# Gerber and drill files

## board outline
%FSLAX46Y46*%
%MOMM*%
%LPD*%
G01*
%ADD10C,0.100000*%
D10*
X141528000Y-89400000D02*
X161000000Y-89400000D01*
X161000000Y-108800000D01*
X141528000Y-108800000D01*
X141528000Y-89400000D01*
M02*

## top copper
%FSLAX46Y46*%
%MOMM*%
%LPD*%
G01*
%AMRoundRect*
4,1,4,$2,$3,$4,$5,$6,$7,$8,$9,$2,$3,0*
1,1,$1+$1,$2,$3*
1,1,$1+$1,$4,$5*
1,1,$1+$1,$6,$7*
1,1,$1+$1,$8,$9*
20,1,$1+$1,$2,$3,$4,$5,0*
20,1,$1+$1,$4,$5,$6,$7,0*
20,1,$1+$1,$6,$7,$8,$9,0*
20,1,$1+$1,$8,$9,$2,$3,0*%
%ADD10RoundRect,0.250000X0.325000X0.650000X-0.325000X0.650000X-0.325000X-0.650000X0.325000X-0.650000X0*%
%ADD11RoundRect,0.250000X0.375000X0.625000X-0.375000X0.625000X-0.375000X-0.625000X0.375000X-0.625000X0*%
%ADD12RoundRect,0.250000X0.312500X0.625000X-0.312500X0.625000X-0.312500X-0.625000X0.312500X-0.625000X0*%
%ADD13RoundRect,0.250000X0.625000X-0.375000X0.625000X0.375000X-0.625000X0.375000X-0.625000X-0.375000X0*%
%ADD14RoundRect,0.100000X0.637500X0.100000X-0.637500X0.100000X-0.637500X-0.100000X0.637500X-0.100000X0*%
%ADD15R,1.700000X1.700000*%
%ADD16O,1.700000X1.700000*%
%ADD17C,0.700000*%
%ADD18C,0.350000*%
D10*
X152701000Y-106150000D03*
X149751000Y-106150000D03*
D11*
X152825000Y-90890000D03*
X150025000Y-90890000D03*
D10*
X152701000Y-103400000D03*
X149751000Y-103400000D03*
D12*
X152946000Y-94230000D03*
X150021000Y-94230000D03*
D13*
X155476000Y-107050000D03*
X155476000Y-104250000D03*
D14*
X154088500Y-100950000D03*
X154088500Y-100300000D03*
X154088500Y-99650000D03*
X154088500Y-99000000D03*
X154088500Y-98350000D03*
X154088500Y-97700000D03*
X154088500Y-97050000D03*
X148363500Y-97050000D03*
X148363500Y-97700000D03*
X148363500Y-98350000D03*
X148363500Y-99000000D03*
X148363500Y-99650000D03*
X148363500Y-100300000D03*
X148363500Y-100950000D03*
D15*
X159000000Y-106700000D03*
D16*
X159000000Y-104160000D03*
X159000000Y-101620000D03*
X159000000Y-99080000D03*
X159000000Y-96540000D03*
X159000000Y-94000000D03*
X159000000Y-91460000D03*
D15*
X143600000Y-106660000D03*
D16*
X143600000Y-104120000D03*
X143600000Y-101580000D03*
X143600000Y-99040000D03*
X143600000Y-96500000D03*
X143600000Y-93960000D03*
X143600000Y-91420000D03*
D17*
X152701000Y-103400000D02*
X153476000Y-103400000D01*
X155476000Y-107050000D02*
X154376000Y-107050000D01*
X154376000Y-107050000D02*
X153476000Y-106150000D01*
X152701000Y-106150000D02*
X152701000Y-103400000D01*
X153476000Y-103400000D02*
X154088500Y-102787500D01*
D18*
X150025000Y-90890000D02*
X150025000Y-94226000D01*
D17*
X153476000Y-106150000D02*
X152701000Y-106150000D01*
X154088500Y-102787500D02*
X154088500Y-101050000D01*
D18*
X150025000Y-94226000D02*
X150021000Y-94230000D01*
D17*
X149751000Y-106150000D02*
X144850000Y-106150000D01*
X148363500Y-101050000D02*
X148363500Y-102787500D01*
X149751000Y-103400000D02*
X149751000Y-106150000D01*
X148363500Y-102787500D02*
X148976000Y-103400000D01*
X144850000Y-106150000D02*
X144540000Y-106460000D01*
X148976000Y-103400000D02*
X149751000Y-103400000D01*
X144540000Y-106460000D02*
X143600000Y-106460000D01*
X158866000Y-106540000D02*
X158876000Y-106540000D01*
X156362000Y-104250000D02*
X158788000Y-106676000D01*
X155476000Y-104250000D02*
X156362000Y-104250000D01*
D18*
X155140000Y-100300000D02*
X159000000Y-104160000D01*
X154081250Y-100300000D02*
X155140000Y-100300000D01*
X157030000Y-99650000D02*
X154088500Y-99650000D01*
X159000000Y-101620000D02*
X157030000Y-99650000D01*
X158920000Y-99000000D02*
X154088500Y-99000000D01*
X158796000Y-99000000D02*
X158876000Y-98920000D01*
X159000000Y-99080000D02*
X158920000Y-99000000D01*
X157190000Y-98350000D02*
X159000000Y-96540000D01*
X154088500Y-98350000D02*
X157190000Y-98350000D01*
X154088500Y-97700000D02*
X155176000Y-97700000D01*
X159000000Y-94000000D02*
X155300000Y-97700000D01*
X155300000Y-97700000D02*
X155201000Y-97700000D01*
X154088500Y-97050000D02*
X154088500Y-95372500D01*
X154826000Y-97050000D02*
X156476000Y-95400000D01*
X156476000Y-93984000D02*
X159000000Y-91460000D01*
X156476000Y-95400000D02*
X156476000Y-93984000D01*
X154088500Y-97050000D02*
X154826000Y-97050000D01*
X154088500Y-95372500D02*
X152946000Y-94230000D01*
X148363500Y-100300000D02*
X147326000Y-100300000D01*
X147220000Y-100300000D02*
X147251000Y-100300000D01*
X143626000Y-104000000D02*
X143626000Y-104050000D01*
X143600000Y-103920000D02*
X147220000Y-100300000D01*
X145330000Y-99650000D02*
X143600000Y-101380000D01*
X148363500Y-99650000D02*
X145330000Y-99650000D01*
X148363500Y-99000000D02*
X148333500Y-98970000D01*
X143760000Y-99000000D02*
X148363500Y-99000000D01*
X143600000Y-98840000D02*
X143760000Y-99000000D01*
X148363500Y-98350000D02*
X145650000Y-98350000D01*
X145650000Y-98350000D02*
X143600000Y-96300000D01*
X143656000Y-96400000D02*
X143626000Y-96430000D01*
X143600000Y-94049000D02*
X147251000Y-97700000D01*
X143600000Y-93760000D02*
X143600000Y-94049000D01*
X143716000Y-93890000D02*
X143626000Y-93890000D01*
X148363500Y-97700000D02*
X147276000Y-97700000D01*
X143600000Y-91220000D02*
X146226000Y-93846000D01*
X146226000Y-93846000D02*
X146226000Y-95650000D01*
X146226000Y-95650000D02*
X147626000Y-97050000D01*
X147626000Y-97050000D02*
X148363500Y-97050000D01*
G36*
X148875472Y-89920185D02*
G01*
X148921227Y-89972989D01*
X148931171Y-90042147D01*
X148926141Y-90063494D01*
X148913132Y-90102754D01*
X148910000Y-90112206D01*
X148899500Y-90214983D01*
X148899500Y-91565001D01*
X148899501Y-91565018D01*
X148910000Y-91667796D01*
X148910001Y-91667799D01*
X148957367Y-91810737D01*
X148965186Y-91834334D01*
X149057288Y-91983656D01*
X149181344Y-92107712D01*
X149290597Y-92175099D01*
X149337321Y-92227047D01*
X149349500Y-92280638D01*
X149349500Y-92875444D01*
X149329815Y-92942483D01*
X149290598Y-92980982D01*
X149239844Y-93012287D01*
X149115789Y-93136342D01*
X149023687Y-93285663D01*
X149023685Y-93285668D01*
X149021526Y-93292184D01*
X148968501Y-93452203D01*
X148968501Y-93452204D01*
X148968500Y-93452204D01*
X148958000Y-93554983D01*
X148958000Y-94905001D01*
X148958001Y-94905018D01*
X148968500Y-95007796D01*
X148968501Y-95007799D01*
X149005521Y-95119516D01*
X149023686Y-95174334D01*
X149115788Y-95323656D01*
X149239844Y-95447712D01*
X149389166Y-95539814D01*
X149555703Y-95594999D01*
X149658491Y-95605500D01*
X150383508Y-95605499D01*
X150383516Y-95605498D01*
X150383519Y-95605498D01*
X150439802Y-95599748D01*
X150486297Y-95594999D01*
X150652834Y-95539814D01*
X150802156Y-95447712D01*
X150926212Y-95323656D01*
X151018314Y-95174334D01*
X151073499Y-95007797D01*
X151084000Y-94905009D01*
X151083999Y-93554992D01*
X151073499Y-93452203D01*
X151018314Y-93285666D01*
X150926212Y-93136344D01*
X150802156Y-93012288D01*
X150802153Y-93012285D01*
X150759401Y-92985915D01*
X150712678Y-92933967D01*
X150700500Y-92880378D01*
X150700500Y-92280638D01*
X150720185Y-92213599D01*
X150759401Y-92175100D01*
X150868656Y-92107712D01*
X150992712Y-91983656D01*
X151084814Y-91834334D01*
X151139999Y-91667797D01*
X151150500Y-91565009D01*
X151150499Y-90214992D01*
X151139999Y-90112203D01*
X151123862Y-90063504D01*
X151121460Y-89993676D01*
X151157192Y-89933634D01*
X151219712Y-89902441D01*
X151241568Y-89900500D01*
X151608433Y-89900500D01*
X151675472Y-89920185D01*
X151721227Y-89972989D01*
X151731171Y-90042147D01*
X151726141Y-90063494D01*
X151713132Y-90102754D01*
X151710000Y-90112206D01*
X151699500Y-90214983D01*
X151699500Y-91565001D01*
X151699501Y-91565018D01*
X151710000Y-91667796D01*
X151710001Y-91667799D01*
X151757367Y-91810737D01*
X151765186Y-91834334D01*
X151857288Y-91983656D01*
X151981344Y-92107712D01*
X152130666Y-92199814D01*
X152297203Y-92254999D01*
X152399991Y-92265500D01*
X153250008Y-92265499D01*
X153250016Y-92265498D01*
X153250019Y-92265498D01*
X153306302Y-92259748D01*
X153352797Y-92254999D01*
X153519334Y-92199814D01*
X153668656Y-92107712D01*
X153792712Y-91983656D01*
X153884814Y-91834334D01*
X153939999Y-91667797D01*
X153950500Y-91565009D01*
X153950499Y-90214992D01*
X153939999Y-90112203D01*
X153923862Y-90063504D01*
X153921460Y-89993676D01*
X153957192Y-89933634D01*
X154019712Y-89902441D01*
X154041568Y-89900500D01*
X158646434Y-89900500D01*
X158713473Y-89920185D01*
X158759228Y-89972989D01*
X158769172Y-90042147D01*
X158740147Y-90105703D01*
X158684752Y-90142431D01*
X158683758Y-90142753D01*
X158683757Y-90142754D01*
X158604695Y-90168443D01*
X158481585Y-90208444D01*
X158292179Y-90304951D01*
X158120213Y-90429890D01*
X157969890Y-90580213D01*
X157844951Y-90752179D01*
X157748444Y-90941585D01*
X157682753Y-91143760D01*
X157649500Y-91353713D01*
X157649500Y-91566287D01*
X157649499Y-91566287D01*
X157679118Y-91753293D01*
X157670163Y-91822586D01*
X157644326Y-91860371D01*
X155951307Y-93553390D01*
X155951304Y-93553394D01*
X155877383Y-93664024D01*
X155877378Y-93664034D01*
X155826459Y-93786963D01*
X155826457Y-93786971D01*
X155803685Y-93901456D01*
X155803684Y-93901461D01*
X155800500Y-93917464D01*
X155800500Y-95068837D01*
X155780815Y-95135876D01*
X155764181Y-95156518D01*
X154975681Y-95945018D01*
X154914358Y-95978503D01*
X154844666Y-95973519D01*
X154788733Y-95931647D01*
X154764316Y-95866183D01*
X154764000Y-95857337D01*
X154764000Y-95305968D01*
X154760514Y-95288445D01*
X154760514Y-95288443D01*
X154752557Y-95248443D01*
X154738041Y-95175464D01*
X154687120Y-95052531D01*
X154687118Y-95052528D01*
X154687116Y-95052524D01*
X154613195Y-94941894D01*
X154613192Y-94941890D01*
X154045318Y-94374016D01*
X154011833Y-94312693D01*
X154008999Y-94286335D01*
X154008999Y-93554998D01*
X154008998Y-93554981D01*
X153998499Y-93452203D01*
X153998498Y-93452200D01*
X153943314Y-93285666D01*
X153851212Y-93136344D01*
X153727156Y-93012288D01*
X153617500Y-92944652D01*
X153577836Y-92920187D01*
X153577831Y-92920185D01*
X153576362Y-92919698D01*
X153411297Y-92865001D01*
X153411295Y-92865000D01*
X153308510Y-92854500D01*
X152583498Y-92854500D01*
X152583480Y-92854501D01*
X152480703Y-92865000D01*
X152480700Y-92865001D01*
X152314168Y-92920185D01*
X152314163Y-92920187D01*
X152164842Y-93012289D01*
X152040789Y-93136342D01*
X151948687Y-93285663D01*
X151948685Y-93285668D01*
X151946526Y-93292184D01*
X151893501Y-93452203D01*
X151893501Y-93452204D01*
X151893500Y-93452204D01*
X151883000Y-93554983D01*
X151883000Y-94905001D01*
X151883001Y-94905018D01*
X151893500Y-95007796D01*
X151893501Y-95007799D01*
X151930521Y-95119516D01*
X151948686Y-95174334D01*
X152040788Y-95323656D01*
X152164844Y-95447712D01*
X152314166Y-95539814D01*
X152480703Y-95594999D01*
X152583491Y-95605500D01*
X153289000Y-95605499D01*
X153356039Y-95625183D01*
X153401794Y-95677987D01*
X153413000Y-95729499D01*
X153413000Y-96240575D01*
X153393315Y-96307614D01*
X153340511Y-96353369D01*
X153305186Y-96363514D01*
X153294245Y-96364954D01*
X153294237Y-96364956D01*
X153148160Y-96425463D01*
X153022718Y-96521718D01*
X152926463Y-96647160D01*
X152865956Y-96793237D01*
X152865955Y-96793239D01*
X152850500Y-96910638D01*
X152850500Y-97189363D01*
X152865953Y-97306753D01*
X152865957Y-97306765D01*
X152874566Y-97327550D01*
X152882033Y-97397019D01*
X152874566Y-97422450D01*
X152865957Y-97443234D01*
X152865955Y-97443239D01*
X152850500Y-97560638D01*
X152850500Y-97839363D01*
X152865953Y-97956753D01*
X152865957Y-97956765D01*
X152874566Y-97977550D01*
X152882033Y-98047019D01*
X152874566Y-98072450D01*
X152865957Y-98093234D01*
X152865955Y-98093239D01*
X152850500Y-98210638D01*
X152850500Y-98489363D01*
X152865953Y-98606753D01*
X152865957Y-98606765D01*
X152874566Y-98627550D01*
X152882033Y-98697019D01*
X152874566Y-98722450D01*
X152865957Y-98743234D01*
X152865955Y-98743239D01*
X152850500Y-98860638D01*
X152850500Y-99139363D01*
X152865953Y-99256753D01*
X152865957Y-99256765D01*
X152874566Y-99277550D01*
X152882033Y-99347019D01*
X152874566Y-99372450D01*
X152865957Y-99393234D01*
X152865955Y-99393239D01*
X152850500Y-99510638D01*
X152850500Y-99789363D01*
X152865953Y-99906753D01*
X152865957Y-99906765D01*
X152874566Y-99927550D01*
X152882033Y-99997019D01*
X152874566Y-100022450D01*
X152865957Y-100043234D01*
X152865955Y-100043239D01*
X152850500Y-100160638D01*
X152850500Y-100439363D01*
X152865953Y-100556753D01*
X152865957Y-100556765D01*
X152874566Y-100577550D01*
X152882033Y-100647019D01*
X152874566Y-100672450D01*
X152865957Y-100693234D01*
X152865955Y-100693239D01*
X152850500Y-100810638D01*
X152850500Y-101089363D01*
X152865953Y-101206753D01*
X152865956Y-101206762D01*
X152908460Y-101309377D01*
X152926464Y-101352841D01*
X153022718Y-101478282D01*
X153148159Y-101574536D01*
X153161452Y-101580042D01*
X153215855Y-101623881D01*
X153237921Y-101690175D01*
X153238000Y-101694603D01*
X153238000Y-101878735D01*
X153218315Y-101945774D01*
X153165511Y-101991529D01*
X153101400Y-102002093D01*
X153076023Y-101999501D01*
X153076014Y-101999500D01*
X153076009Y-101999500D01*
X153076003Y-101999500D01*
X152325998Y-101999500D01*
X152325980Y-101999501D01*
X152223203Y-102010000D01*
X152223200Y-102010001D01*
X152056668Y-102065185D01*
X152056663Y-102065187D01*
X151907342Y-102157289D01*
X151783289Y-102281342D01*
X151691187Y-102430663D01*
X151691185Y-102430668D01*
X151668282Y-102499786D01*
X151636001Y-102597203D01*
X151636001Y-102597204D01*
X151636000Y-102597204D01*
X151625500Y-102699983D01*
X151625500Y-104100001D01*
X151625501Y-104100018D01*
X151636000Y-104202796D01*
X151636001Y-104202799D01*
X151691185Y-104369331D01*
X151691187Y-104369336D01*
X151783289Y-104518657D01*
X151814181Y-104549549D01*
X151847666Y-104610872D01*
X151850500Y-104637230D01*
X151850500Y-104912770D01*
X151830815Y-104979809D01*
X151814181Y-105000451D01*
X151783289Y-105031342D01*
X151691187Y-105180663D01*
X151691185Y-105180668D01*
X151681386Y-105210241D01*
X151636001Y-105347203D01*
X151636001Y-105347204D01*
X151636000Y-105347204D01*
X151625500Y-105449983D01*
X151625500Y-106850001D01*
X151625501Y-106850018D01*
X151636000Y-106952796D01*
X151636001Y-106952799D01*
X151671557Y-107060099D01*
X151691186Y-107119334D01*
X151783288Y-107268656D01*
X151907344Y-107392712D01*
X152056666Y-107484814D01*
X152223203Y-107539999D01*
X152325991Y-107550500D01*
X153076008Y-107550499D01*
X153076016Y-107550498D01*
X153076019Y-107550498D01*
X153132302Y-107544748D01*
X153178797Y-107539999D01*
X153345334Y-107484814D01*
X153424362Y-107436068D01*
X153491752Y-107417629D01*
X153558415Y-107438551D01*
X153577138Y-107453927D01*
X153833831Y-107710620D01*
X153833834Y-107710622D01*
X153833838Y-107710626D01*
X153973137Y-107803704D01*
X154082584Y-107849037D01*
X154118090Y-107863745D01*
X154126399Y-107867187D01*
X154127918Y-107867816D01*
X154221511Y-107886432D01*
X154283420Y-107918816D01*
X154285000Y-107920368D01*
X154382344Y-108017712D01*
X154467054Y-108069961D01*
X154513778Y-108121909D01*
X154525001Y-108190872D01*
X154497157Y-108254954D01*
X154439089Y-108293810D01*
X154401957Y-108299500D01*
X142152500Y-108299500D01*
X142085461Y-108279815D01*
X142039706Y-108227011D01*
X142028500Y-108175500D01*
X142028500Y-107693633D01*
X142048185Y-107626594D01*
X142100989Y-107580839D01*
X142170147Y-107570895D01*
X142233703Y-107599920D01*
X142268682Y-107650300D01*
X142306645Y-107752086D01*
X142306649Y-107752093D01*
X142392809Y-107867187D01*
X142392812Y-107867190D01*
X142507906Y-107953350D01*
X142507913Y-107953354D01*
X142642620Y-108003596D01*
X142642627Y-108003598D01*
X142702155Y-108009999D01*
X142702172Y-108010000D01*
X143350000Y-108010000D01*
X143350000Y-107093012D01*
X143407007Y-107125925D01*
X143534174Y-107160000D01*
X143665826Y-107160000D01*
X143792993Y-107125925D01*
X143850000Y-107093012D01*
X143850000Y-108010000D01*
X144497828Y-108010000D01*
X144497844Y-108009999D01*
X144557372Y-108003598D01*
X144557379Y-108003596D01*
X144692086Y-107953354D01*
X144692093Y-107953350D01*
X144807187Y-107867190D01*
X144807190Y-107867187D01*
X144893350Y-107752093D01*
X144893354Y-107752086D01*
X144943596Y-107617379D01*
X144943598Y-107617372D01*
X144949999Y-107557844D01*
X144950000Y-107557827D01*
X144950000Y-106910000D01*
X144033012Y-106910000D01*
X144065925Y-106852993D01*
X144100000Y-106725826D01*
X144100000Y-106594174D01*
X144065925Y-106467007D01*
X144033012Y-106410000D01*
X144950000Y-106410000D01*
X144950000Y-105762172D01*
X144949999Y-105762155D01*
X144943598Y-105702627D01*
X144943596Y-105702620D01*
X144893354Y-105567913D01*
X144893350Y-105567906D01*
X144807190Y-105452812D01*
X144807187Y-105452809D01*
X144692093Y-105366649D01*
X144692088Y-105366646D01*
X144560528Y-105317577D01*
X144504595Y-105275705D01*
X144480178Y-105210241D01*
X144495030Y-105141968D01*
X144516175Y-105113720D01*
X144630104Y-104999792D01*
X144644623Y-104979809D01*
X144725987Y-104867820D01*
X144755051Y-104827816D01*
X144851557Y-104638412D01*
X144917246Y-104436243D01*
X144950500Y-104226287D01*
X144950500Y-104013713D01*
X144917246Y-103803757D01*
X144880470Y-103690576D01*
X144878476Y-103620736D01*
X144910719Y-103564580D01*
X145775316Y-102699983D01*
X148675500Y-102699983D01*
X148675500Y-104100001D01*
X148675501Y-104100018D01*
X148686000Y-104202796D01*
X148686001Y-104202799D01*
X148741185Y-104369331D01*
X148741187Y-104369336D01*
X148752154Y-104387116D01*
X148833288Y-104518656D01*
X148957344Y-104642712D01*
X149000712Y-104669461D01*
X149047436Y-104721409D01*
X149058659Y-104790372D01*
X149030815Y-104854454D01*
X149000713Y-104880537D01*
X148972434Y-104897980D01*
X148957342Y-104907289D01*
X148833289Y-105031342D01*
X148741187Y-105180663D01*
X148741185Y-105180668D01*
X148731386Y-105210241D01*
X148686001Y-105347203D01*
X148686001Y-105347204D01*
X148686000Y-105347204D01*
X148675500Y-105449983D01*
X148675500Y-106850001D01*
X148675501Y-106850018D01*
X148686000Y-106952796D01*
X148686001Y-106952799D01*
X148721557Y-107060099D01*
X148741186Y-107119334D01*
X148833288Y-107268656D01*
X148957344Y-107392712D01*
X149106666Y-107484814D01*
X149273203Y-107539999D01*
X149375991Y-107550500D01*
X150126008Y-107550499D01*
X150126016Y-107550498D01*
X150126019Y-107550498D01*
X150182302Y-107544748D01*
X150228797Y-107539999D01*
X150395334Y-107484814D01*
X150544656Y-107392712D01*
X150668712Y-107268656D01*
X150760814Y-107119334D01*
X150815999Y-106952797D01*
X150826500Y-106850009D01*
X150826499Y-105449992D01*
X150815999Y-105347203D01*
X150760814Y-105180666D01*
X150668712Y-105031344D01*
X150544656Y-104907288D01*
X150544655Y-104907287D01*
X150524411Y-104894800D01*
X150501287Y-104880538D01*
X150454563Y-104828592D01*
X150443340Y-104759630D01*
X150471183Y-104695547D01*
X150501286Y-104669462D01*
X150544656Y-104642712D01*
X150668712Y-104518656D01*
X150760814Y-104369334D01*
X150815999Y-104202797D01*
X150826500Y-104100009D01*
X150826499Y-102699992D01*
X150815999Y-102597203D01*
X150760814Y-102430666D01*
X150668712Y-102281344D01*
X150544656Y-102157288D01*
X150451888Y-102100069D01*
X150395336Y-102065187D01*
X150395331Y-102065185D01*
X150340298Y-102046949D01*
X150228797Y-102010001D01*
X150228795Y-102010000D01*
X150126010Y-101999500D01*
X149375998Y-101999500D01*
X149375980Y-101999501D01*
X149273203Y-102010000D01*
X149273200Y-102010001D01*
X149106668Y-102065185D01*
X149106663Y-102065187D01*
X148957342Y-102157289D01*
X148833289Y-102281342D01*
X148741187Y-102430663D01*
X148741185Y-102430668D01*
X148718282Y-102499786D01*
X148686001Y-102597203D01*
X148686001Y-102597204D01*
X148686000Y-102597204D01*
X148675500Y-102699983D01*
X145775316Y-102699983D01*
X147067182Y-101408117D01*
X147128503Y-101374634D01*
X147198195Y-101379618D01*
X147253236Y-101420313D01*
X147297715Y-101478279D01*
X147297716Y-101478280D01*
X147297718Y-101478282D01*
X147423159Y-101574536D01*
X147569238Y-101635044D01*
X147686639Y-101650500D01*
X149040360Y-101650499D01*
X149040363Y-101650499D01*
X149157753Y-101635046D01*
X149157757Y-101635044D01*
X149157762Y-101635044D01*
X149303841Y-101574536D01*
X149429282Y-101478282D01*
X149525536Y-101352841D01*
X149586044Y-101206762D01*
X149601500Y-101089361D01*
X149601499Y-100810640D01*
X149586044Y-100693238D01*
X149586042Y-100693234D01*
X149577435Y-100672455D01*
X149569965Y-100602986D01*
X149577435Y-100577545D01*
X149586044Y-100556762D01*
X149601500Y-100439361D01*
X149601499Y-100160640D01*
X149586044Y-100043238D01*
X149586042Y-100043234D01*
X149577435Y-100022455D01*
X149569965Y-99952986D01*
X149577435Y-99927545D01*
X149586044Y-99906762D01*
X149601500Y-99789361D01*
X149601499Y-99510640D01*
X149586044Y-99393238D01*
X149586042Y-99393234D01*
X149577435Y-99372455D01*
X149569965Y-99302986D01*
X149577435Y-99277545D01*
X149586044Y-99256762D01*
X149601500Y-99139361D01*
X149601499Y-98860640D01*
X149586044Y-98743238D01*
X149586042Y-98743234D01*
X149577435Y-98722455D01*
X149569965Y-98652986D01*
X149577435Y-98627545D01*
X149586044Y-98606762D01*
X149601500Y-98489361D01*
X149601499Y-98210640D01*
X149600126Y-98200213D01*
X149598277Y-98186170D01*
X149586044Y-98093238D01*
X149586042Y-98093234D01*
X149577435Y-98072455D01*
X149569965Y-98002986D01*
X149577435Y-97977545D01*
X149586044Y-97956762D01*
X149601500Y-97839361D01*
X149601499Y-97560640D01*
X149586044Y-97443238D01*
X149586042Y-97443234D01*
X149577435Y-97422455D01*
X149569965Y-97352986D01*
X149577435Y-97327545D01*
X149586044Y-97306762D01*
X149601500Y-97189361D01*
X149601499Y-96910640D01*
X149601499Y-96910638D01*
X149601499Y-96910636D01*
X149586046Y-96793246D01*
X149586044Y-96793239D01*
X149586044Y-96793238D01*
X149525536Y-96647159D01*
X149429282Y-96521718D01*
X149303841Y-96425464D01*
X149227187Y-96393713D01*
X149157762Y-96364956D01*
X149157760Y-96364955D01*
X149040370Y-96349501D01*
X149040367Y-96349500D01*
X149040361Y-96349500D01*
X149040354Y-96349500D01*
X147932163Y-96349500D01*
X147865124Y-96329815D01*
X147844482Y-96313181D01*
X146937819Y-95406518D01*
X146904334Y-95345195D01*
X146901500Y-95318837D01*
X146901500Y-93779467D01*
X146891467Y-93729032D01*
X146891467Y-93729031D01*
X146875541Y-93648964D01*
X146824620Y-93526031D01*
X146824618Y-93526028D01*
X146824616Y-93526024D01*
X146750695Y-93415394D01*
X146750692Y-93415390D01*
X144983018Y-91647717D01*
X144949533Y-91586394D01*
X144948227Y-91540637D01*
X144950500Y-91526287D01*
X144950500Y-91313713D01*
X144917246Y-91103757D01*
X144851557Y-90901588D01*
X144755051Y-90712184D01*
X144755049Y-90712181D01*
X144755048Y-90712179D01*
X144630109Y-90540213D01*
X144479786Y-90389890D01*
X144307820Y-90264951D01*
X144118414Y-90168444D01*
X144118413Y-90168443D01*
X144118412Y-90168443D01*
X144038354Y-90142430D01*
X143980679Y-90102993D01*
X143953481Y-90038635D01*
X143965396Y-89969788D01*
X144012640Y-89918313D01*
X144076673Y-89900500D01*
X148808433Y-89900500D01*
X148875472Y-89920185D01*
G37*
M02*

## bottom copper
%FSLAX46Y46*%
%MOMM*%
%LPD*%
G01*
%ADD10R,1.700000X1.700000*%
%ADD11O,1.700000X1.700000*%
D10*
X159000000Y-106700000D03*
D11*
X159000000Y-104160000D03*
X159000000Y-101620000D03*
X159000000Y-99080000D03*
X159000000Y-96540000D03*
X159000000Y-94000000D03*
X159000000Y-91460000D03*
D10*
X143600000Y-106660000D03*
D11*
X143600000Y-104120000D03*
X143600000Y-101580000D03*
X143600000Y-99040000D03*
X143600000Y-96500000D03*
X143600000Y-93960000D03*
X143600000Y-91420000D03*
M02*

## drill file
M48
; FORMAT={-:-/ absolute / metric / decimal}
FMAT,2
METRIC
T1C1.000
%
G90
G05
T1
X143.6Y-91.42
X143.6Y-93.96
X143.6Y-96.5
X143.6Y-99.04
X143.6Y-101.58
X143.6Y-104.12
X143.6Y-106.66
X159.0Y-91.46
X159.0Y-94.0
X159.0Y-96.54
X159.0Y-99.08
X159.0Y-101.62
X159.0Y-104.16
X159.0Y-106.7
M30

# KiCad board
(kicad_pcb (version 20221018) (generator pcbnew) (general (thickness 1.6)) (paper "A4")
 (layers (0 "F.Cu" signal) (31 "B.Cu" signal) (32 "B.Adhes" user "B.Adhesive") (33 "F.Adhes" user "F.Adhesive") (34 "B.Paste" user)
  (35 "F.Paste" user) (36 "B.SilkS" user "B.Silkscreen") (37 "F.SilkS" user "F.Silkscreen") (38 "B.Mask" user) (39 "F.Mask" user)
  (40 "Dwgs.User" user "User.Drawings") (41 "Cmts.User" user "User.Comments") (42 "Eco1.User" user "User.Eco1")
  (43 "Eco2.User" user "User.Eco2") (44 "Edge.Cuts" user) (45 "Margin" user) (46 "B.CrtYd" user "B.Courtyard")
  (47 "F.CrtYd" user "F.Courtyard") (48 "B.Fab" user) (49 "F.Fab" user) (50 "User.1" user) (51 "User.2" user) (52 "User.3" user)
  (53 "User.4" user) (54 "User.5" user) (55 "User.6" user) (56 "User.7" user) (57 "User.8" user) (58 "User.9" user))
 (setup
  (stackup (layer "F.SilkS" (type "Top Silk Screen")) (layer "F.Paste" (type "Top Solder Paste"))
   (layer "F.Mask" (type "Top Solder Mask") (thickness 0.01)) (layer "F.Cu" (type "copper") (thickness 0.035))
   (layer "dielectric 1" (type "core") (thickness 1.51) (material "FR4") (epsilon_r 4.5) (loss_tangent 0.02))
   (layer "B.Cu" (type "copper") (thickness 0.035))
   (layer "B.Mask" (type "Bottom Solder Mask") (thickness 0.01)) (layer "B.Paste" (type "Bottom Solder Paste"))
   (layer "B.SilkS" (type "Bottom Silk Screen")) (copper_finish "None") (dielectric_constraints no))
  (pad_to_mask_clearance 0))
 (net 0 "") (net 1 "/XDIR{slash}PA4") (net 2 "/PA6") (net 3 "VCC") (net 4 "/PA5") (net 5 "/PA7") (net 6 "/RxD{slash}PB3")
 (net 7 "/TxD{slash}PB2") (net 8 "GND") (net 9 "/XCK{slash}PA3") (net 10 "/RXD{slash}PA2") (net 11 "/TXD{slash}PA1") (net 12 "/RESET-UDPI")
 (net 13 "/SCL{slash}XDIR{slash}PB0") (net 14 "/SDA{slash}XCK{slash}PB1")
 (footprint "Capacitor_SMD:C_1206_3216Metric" (layer "F.Cu") (at 151.226 106.15 180)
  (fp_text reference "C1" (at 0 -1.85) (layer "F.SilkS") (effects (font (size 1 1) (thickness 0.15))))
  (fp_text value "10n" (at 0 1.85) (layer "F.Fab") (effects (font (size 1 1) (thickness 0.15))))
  (pad "1" smd roundrect (at -1.475 0 180) (size 1.15 1.8) (layers "F.Cu" "F.Paste" "F.Mask") (roundrect_rratio 0.2173913043))
  (pad "2" smd roundrect (at 1.475 0 180) (size 1.15 1.8) (layers "F.Cu" "F.Paste" "F.Mask") (roundrect_rratio 0.2173913043)))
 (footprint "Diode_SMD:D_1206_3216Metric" (layer "F.Cu") (at 151.425 90.89 180)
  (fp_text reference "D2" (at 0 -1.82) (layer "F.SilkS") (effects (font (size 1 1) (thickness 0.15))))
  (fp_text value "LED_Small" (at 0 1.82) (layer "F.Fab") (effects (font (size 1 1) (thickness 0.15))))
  (pad "1" smd roundrect (at -1.4 0 180) (size 1.25 1.75) (layers "F.Cu" "F.Paste" "F.Mask") (roundrect_rratio 0.2))
  (pad "2" smd roundrect (at 1.4 0 180) (size 1.25 1.75) (layers "F.Cu" "F.Paste" "F.Mask") (roundrect_rratio 0.2)))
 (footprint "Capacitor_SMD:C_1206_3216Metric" (layer "F.Cu") (at 151.226 103.4 180)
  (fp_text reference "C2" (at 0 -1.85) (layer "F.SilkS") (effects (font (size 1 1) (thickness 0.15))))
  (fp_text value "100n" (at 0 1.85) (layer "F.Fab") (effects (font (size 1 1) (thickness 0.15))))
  (pad "1" smd roundrect (at -1.475 0 180) (size 1.15 1.8) (layers "F.Cu" "F.Paste" "F.Mask") (roundrect_rratio 0.2173913043))
  (pad "2" smd roundrect (at 1.475 0 180) (size 1.15 1.8) (layers "F.Cu" "F.Paste" "F.Mask") (roundrect_rratio 0.2173913043)))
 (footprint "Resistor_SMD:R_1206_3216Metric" (layer "F.Cu") (at 151.4835 94.23 180)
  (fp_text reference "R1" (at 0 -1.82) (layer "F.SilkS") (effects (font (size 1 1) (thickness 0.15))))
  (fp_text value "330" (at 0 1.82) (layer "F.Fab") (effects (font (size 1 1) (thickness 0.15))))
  (pad "1" smd roundrect (at -1.4625 0 180) (size 1.125 1.75) (layers "F.Cu" "F.Paste" "F.Mask") (roundrect_rratio 0.2222222222))
  (pad "2" smd roundrect (at 1.4625 0 180) (size 1.125 1.75) (layers "F.Cu" "F.Paste" "F.Mask") (roundrect_rratio 0.2222222222)))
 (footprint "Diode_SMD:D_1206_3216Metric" (layer "F.Cu") (at 155.476 105.65 90)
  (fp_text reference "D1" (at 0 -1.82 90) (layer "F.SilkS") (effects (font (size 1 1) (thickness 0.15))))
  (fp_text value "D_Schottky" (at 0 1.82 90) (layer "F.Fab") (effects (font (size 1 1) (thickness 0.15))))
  (pad "1" smd roundrect (at -1.4 0 90) (size 1.25 1.75) (layers "F.Cu" "F.Paste" "F.Mask") (roundrect_rratio 0.2))
  (pad "2" smd roundrect (at 1.4 0 90) (size 1.25 1.75) (layers "F.Cu" "F.Paste" "F.Mask") (roundrect_rratio 0.2)))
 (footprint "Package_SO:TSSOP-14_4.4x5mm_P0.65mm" (layer "F.Cu") (at 151.226 99 180)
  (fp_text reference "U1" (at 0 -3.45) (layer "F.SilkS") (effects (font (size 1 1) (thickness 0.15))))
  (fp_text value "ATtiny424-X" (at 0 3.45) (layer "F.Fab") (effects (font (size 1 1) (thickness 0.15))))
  (pad "1" smd roundrect (at -2.8625 -1.95 180) (size 1.475 0.4) (layers "F.Cu" "F.Paste" "F.Mask") (roundrect_rratio 0.25))
  (pad "2" smd roundrect (at -2.8625 -1.3 180) (size 1.475 0.4) (layers "F.Cu" "F.Paste" "F.Mask") (roundrect_rratio 0.25)
   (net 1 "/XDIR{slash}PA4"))
  (pad "3" smd roundrect (at -2.8625 -0.65 180) (size 1.475 0.4) (layers "F.Cu" "F.Paste" "F.Mask") (roundrect_rratio 0.25))
  (pad "4" smd roundrect (at -2.8625 0 180) (size 1.475 0.4) (layers "F.Cu" "F.Paste" "F.Mask") (roundrect_rratio 0.25) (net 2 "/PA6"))
  (pad "5" smd roundrect (at -2.8625 0.65 180) (size 1.475 0.4) (layers "F.Cu" "F.Paste" "F.Mask") (roundrect_rratio 0.25))
  (pad "6" smd roundrect (at -2.8625 1.3 180) (size 1.475 0.4) (layers "F.Cu" "F.Paste" "F.Mask") (roundrect_rratio 0.25))
  (pad "7" smd roundrect (at -2.8625 1.95 180) (size 1.475 0.4) (layers "F.Cu" "F.Paste" "F.Mask") (roundrect_rratio 0.25))
  (pad "8" smd roundrect (at 2.8625 1.95 180) (size 1.475 0.4) (layers "F.Cu" "F.Paste" "F.Mask") (roundrect_rratio 0.25))
  (pad "9" smd roundrect (at 2.8625 1.3 180) (size 1.475 0.4) (layers "F.Cu" "F.Paste" "F.Mask") (roundrect_rratio 0.25))
  (pad "10" smd roundrect (at 2.8625 0.65 180) (size 1.475 0.4) (layers "F.Cu" "F.Paste" "F.Mask") (roundrect_rratio 0.25))
  (pad "11" smd roundrect (at 2.8625 0 180) (size 1.475 0.4) (layers "F.Cu" "F.Paste" "F.Mask") (roundrect_rratio 0.25))
  (pad "12" smd roundrect (at 2.8625 -0.65 180) (size 1.475 0.4) (layers "F.Cu" "F.Paste" "F.Mask") (roundrect_rratio 0.25))
  (pad "13" smd roundrect (at 2.8625 -1.3 180) (size 1.475 0.4) (layers "F.Cu" "F.Paste" "F.Mask") (roundrect_rratio 0.25))
  (pad "14" smd roundrect (at 2.8625 -1.95 180) (size 1.475 0.4) (layers "F.Cu" "F.Paste" "F.Mask") (roundrect_rratio 0.25)))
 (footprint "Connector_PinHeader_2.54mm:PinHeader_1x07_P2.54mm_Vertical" (layer "B.Cu") (at 159 106.7)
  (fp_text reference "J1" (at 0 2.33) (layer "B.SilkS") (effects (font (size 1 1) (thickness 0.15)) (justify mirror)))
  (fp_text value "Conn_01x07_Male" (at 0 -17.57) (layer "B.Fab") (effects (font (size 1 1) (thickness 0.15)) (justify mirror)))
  (pad "1" thru_hole rect (at 0 0) (size 1.7 1.7) (drill 1) (layers "*.Cu" "*.Mask") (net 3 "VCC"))
  (pad "2" thru_hole oval (at 0 -2.54) (size 1.7 1.7) (drill 1) (layers "*.Cu" "*.Mask") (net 1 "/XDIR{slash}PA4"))
  (pad "3" thru_hole oval (at 0 -5.08) (size 1.7 1.7) (drill 1) (layers "*.Cu" "*.Mask") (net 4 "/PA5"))
  (pad "4" thru_hole oval (at 0 -7.62) (size 1.7 1.7) (drill 1) (layers "*.Cu" "*.Mask") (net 2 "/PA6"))
  (pad "5" thru_hole oval (at 0 -10.16) (size 1.7 1.7) (drill 1) (layers "*.Cu" "*.Mask") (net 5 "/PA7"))
  (pad "6" thru_hole oval (at 0 -12.7) (size 1.7 1.7) (drill 1) (layers "*.Cu" "*.Mask") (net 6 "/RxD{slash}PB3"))
  (pad "7" thru_hole oval (at 0 -15.24) (size 1.7 1.7) (drill 1) (layers "*.Cu" "*.Mask") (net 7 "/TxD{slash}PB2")))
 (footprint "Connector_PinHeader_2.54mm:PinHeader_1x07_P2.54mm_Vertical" (layer "B.Cu") (at 143.6 106.66)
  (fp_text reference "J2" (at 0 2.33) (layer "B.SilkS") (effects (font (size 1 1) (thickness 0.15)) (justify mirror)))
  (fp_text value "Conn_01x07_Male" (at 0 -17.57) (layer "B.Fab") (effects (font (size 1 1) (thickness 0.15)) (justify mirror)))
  (pad "1" thru_hole rect (at 0 0) (size 1.7 1.7) (drill 1) (layers "*.Cu" "*.Mask") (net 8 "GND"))
  (pad "2" thru_hole oval (at 0 -2.54) (size 1.7 1.7) (drill 1) (layers "*.Cu" "*.Mask") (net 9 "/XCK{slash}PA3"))
  (pad "3" thru_hole oval (at 0 -5.08) (size 1.7 1.7) (drill 1) (layers "*.Cu" "*.Mask") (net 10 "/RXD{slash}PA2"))
  (pad "4" thru_hole oval (at 0 -7.62) (size 1.7 1.7) (drill 1) (layers "*.Cu" "*.Mask") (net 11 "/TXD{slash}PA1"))
  (pad "5" thru_hole oval (at 0 -10.16) (size 1.7 1.7) (drill 1) (layers "*.Cu" "*.Mask") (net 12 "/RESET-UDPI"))
  (pad "6" thru_hole oval (at 0 -12.7) (size 1.7 1.7) (drill 1) (layers "*.Cu" "*.Mask") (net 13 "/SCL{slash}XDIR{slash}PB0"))
  (pad "7" thru_hole oval (at 0 -15.24) (size 1.7 1.7) (drill 1) (layers "*.Cu" "*.Mask") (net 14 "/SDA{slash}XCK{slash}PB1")))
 (gr_rect (start 141.528 89.4) (end 161 108.8) (stroke (width 0.1) (type solid)) (fill none) (layer "Edge.Cuts"))
 (segment (start 152.701 103.4) (end 153.476 103.4) (width 0.7) (layer "F.Cu") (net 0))
 (segment (start 155.476 107.05) (end 154.376 107.05) (width 0.7) (layer "F.Cu") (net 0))
 (segment (start 154.376 107.05) (end 153.476 106.15) (width 0.7) (layer "F.Cu") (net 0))
 (segment (start 152.701 106.15) (end 152.701 103.4) (width 0.7) (layer "F.Cu") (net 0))
 (segment (start 153.476 103.4) (end 154.0885 102.7875) (width 0.7) (layer "F.Cu") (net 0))
 (segment (start 150.025 90.89) (end 150.025 94.226) (width 0.35) (layer "F.Cu") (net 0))
 (segment (start 153.476 106.15) (end 152.701 106.15) (width 0.7) (layer "F.Cu") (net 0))
 (segment (start 154.0885 102.7875) (end 154.0885 101.05) (width 0.7) (layer "F.Cu") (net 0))
 (segment (start 150.025 94.226) (end 150.021 94.23) (width 0.35) (layer "F.Cu") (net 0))
 (segment (start 149.751 106.15) (end 144.85 106.15) (width 0.7) (layer "F.Cu") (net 8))
 (segment (start 148.3635 101.05) (end 148.3635 102.7875) (width 0.7) (layer "F.Cu") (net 8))
 (segment (start 149.751 103.4) (end 149.751 106.15) (width 0.7) (layer "F.Cu") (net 8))
 (segment (start 148.3635 102.7875) (end 148.976 103.4) (width 0.7) (layer "F.Cu") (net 8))
 (segment (start 144.85 106.15) (end 144.54 106.46) (width 0.7) (layer "F.Cu") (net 8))
 (segment (start 148.976 103.4) (end 149.751 103.4) (width 0.7) (layer "F.Cu") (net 8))
 (segment (start 144.54 106.46) (end 143.6 106.46) (width 0.7) (layer "F.Cu") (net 8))
 (segment (start 158.866 106.54) (end 158.876 106.54) (width 0.7) (layer "F.Cu") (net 3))
 (segment (start 156.362 104.25) (end 158.788 106.676) (width 0.7) (layer "F.Cu") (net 3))
 (segment (start 155.476 104.25) (end 156.362 104.25) (width 0.7) (layer "F.Cu") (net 3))
 (segment (start 155.14 100.3) (end 159 104.16) (width 0.35) (layer "F.Cu") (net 1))
 (segment (start 154.08125 100.3) (end 155.14 100.3) (width 0.35) (layer "F.Cu") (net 1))
 (segment (start 157.03 99.65) (end 154.0885 99.65) (width 0.35) (layer "F.Cu") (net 4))
 (segment (start 159 101.62) (end 157.03 99.65) (width 0.35) (layer "F.Cu") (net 4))
 (segment (start 158.92 99) (end 154.0885 99) (width 0.35) (layer "F.Cu") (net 2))
 (segment (start 158.796 99) (end 158.876 98.92) (width 0.35) (layer "F.Cu") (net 2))
 (segment (start 159 99.08) (end 158.92 99) (width 0.35) (layer "F.Cu") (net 2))
 (segment (start 157.19 98.35) (end 159 96.54) (width 0.35) (layer "F.Cu") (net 5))
 (segment (start 154.0885 98.35) (end 157.19 98.35) (width 0.35) (layer "F.Cu") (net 5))
 (segment (start 154.0885 97.7) (end 155.176 97.7) (width 0.35) (layer "F.Cu") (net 6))
 (segment (start 159 94) (end 155.3 97.7) (width 0.35) (layer "F.Cu") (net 6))
 (segment (start 155.3 97.7) (end 155.201 97.7) (width 0.35) (layer "F.Cu") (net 6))
 (segment (start 154.0885 97.05) (end 154.0885 95.3725) (width 0.35) (layer "F.Cu") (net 7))
 (segment (start 154.826 97.05) (end 156.476 95.4) (width 0.35) (layer "F.Cu") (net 7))
 (segment (start 156.476 93.984) (end 159 91.46) (width 0.35) (layer "F.Cu") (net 7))
 (segment (start 156.476 95.4) (end 156.476 93.984) (width 0.35) (layer "F.Cu") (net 7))
 (segment (start 154.0885 97.05) (end 154.826 97.05) (width 0.35) (layer "F.Cu") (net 7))
 (segment (start 154.0885 95.3725) (end 152.946 94.23) (width 0.35) (layer "F.Cu") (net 7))
 (segment (start 148.3635 100.3) (end 147.326 100.3) (width 0.35) (layer "F.Cu") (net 9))
 (segment (start 147.22 100.3) (end 147.251 100.3) (width 0.35) (layer "F.Cu") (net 9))
 (segment (start 143.626 104) (end 143.626 104.05) (width 0.35) (layer "F.Cu") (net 9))
 (segment (start 143.6 103.92) (end 147.22 100.3) (width 0.35) (layer "F.Cu") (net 9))
 (segment (start 145.33 99.65) (end 143.6 101.38) (width 0.35) (layer "F.Cu") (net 10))
 (segment (start 148.3635 99.65) (end 145.33 99.65) (width 0.35) (layer "F.Cu") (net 10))
 (segment (start 148.3635 99) (end 148.3335 98.97) (width 0.35) (layer "F.Cu") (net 11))
 (segment (start 143.76 99) (end 148.3635 99) (width 0.35) (layer "F.Cu") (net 11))
 (segment (start 143.6 98.84) (end 143.76 99) (width 0.35) (layer "F.Cu") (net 11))
 (segment (start 148.3635 98.35) (end 145.65 98.35) (width 0.35) (layer "F.Cu") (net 12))
 (segment (start 145.65 98.35) (end 143.6 96.3) (width 0.35) (layer "F.Cu") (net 12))
 (segment (start 143.656 96.4) (end 143.626 96.43) (width 0.35) (layer "F.Cu") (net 12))
 (segment (start 143.6 94.049) (end 147.251 97.7) (width 0.35) (layer "F.Cu") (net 13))
 (segment (start 143.6 93.76) (end 143.6 94.049) (width 0.35) (layer "F.Cu") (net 13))
 (segment (start 143.716 93.89) (end 143.626 93.89) (width 0.35) (layer "F.Cu") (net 13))
 (segment (start 148.3635 97.7) (end 147.276 97.7) (width 0.35) (layer "F.Cu") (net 13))
 (segment (start 143.6 91.22) (end 146.226 93.846) (width 0.35) (layer "F.Cu") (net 14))
 (segment (start 146.226 93.846) (end 146.226 95.65) (width 0.35) (layer "F.Cu") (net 14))
 (segment (start 146.226 95.65) (end 147.626 97.05) (width 0.35) (layer "F.Cu") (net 14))
 (segment (start 147.626 97.05) (end 148.3635 97.05) (width 0.35) (layer "F.Cu") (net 14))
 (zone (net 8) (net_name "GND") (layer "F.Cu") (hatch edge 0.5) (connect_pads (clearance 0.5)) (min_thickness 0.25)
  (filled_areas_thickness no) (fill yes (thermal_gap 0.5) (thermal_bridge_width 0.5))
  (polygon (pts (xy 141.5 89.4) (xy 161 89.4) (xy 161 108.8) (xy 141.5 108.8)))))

